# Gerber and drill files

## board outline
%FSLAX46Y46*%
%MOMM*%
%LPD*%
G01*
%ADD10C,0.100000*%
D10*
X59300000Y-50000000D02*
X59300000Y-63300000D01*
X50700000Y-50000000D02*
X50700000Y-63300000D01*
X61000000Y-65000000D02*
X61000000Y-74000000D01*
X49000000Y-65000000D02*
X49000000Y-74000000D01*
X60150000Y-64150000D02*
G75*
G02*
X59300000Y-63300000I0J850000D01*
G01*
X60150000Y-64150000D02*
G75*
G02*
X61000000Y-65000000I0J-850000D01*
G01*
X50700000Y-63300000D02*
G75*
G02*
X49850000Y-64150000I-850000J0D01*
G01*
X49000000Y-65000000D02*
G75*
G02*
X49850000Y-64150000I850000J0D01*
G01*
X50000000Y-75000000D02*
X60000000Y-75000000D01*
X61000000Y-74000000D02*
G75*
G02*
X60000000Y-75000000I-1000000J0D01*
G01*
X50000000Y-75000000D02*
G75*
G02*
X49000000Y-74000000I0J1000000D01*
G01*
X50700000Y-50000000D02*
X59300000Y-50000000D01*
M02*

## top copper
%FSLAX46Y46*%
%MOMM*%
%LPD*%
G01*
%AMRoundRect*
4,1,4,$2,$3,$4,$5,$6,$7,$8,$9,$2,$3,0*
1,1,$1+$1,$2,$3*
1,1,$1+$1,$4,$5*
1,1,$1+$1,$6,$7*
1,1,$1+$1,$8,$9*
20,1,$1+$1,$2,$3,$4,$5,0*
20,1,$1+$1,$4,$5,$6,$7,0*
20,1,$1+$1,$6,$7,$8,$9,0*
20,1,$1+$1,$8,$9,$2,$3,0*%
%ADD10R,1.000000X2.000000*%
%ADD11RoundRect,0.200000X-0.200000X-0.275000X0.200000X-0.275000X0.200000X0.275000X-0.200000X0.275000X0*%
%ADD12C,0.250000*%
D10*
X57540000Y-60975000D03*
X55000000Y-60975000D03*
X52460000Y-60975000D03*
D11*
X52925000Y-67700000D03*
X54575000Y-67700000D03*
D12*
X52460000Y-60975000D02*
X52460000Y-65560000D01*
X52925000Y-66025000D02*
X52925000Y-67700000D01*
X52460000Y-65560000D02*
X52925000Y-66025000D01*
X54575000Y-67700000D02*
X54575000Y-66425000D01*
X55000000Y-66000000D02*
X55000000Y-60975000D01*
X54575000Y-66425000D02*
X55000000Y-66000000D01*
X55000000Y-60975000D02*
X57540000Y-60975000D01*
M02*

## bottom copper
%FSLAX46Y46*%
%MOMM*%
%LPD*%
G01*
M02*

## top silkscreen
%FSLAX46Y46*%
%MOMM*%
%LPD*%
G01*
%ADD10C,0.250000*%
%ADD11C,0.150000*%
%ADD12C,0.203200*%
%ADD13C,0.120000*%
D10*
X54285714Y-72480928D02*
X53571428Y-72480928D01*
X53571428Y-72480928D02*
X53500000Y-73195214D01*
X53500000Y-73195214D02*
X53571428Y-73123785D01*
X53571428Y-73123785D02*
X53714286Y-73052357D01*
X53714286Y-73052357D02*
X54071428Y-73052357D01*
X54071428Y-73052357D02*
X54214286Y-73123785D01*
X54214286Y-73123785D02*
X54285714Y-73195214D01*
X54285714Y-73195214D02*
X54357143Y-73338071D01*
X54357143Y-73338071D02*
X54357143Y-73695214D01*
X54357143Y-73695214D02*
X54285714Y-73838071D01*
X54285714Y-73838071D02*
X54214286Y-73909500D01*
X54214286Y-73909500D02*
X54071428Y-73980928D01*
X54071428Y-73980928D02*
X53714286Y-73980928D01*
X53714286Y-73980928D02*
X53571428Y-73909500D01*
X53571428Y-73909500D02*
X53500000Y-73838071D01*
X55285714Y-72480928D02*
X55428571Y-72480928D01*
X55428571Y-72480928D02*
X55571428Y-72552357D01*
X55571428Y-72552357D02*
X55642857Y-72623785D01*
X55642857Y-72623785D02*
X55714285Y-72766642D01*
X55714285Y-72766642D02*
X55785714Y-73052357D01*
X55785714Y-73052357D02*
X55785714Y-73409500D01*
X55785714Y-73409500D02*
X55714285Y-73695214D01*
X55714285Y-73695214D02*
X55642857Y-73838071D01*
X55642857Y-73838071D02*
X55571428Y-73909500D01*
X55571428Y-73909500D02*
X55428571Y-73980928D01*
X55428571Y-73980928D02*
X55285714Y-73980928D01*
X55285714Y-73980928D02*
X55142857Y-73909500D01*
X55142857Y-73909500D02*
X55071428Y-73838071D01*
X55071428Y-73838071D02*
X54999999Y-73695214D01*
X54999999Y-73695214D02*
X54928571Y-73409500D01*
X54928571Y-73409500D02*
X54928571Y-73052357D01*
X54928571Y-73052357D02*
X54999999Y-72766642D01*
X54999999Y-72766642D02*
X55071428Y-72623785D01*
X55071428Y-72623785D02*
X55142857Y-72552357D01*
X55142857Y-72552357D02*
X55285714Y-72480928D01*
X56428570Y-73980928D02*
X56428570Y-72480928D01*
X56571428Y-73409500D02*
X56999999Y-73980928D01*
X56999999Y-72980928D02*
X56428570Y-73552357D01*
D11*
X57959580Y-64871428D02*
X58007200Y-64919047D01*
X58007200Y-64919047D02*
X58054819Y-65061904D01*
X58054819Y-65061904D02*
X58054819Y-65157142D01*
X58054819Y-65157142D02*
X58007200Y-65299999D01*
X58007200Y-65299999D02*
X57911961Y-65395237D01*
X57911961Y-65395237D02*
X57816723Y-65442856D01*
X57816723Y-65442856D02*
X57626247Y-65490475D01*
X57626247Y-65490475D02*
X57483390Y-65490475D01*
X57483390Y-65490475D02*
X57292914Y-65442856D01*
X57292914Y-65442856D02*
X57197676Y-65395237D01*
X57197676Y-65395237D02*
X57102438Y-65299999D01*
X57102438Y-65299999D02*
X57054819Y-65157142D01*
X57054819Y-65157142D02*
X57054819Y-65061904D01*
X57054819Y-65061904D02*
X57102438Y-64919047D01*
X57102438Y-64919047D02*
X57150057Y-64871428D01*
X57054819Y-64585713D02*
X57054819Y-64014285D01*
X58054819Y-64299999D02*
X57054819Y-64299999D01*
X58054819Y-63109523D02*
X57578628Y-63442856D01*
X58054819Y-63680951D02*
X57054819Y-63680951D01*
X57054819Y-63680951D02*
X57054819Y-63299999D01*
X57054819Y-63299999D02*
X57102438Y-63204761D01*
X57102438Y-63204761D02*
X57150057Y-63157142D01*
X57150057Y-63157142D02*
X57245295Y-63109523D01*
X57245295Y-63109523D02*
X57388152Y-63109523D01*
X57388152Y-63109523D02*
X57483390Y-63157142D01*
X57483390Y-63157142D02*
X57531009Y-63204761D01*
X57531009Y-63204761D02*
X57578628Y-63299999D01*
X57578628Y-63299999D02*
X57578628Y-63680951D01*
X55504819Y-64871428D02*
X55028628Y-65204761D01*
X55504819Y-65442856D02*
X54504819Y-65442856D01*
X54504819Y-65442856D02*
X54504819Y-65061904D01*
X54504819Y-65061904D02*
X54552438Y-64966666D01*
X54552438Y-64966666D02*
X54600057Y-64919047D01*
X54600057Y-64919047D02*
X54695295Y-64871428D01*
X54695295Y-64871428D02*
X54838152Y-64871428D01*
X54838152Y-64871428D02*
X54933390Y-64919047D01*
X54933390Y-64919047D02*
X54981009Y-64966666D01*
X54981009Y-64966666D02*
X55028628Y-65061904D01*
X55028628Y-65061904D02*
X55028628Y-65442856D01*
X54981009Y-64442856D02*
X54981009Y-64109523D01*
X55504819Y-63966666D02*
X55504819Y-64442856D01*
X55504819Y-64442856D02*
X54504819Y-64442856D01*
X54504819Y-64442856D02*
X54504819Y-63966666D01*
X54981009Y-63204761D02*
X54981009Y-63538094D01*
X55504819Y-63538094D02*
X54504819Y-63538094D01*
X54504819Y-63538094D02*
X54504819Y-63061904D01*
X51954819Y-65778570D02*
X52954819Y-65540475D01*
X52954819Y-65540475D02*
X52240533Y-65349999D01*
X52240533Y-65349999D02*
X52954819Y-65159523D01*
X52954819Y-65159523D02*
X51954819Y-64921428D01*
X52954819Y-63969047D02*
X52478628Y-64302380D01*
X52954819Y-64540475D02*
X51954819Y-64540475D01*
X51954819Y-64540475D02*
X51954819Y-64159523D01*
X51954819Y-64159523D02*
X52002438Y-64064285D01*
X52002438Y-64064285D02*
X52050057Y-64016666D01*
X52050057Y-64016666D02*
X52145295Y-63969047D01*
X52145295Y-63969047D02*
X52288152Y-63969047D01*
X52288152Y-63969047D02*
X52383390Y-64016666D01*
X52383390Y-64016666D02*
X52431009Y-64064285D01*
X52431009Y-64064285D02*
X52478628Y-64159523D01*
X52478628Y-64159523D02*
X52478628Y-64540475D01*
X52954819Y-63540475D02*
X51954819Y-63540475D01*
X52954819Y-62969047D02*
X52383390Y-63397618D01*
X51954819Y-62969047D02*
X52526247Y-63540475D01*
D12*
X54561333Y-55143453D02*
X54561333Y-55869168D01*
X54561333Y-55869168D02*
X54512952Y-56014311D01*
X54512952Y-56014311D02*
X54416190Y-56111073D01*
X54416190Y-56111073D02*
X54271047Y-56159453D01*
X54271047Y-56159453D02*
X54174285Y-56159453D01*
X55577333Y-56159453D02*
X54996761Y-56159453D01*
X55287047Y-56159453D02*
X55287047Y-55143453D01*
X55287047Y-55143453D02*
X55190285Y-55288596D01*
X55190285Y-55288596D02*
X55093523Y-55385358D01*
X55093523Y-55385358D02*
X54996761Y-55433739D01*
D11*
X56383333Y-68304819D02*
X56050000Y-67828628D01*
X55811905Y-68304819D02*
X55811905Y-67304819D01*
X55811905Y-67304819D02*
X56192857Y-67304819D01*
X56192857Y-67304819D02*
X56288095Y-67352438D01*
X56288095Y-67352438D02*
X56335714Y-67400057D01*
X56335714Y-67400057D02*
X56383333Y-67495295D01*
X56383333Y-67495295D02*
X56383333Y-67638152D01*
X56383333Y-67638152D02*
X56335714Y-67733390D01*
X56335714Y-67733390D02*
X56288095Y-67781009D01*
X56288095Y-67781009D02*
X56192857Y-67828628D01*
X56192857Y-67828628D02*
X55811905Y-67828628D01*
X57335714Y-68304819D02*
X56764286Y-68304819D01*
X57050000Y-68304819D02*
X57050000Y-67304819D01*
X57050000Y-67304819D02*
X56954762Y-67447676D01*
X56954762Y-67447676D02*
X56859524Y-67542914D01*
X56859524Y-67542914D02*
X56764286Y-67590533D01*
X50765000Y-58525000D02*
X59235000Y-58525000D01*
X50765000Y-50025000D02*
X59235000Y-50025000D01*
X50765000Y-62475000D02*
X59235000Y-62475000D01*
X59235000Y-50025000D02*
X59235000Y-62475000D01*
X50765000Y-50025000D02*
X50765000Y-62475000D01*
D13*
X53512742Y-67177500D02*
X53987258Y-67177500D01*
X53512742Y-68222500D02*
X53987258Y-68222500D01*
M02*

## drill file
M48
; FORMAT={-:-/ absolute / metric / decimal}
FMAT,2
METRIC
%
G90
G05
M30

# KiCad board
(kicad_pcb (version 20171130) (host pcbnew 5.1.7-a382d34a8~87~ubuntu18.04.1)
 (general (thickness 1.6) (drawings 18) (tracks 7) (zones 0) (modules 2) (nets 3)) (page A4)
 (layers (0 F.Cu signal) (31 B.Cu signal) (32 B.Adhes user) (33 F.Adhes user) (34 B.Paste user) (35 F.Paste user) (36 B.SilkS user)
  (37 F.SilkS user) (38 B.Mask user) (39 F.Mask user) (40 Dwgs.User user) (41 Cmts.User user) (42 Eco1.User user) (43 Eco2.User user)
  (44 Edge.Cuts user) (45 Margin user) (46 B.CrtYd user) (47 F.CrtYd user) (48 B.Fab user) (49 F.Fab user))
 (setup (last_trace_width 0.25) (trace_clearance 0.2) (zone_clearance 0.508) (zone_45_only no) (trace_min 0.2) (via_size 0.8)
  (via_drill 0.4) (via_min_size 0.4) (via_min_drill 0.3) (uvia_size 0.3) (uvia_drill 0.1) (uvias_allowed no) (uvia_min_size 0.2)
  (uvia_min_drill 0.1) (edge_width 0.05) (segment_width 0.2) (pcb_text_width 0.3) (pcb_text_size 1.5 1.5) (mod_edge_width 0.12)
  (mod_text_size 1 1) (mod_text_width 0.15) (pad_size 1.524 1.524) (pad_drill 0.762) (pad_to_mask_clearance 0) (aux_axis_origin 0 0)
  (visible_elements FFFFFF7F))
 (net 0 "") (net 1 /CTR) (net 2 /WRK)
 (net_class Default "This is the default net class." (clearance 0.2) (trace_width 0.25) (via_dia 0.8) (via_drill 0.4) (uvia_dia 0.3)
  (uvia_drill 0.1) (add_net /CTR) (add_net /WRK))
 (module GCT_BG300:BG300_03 (layer F.Cu) (at 55 56.25)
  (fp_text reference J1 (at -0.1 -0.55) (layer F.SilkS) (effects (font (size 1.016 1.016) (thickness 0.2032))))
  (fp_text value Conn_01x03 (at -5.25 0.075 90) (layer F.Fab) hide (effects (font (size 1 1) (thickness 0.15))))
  (fp_line (start -4.235 2.275) (end 4.235 2.275) (layer F.SilkS) (width 0.15))
  (fp_line (start -4.235 -6.225) (end 4.235 -6.225) (layer F.SilkS) (width 0.15))
  (fp_line (start -4.235 6.225) (end 4.235 6.225) (layer F.SilkS) (width 0.15))
  (fp_line (start 4.235 -6.225) (end 4.235 6.225) (layer F.SilkS) (width 0.15))
  (fp_line (start -4.235 -6.225) (end -4.235 6.225) (layer F.SilkS) (width 0.15))
  (pad 3 smd rect (at 2.54 4.725) (size 1 2) (layers F.Cu F.Paste F.Mask) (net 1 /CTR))
  (pad 2 smd rect (at 0 4.725) (size 1 2) (layers F.Cu F.Paste F.Mask) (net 1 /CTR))
  (pad 1 smd rect (at -2.54 4.725) (size 1 2) (layers F.Cu F.Paste F.Mask) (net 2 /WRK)))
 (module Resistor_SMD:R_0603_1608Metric (layer F.Cu) (at 53.75 67.7)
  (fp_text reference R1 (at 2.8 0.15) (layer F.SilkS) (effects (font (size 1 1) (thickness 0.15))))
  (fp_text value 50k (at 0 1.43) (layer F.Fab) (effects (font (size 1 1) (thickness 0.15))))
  (fp_line (start -0.237258 -0.5225) (end 0.237258 -0.5225) (layer F.SilkS) (width 0.12))
  (fp_line (start -0.237258 0.5225) (end 0.237258 0.5225) (layer F.SilkS) (width 0.12))
  (pad 1 smd roundrect (at -0.825 0) (size 0.8 0.95) (layers F.Cu F.Paste F.Mask) (roundrect_rratio 0.25) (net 2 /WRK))
  (pad 2 smd roundrect (at 0.825 0) (size 0.8 0.95) (layers F.Cu F.Paste F.Mask) (roundrect_rratio 0.25) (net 1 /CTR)))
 (gr_line (start 59.3 50) (end 59.3 63.3) (layer Edge.Cuts) (width 0.1))
 (gr_line (start 50.7 50) (end 50.7 63.3) (layer Edge.Cuts) (width 0.1))
 (gr_line (start 61 65) (end 61 74) (layer Edge.Cuts) (width 0.1))
 (gr_line (start 49 65) (end 49 74) (layer Edge.Cuts) (width 0.1))
 (gr_arc (start 60.15 63.3) (end 59.3 63.3) (angle -90) (layer Edge.Cuts) (width 0.1))
 (gr_arc (start 60.15 65) (end 61 65) (angle -90) (layer Edge.Cuts) (width 0.1))
 (gr_arc (start 49.85 63.3) (end 49.85 64.15) (angle -90) (layer Edge.Cuts) (width 0.1))
 (gr_arc (start 49.85 65) (end 49.85 64.15) (angle -90) (layer Edge.Cuts) (width 0.1))
 (gr_line (start 50 75) (end 60 75) (layer Edge.Cuts) (width 0.1))
 (gr_arc (start 60 74) (end 60 75) (angle -90) (layer Edge.Cuts) (width 0.1))
 (gr_arc (start 50 74) (end 49 74) (angle -90) (layer Edge.Cuts) (width 0.1))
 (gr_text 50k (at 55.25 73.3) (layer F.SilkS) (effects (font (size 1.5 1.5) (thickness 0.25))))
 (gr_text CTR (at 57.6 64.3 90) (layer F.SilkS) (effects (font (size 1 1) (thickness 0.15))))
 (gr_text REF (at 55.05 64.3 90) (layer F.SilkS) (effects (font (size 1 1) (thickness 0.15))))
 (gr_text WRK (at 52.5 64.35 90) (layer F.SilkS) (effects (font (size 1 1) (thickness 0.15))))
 (gr_line (start 50.7 50) (end 59.3 50) (layer Edge.Cuts) (width 0.1))
 (segment (start 52.46 60.975) (end 52.46 65.56) (width 0.25) (layer F.Cu) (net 2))
 (segment (start 52.925 66.025) (end 52.925 67.7) (width 0.25) (layer F.Cu) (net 2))
 (segment (start 52.46 65.56) (end 52.925 66.025) (width 0.25) (layer F.Cu) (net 2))
 (segment (start 54.575 67.7) (end 54.575 66.425) (width 0.25) (layer F.Cu) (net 1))
 (segment (start 55 66) (end 55 60.975) (width 0.25) (layer F.Cu) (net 1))
 (segment (start 54.575 66.425) (end 55 66) (width 0.25) (layer F.Cu) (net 1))
 (segment (start 55 60.975) (end 57.54 60.975) (width 0.25) (layer F.Cu) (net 1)))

